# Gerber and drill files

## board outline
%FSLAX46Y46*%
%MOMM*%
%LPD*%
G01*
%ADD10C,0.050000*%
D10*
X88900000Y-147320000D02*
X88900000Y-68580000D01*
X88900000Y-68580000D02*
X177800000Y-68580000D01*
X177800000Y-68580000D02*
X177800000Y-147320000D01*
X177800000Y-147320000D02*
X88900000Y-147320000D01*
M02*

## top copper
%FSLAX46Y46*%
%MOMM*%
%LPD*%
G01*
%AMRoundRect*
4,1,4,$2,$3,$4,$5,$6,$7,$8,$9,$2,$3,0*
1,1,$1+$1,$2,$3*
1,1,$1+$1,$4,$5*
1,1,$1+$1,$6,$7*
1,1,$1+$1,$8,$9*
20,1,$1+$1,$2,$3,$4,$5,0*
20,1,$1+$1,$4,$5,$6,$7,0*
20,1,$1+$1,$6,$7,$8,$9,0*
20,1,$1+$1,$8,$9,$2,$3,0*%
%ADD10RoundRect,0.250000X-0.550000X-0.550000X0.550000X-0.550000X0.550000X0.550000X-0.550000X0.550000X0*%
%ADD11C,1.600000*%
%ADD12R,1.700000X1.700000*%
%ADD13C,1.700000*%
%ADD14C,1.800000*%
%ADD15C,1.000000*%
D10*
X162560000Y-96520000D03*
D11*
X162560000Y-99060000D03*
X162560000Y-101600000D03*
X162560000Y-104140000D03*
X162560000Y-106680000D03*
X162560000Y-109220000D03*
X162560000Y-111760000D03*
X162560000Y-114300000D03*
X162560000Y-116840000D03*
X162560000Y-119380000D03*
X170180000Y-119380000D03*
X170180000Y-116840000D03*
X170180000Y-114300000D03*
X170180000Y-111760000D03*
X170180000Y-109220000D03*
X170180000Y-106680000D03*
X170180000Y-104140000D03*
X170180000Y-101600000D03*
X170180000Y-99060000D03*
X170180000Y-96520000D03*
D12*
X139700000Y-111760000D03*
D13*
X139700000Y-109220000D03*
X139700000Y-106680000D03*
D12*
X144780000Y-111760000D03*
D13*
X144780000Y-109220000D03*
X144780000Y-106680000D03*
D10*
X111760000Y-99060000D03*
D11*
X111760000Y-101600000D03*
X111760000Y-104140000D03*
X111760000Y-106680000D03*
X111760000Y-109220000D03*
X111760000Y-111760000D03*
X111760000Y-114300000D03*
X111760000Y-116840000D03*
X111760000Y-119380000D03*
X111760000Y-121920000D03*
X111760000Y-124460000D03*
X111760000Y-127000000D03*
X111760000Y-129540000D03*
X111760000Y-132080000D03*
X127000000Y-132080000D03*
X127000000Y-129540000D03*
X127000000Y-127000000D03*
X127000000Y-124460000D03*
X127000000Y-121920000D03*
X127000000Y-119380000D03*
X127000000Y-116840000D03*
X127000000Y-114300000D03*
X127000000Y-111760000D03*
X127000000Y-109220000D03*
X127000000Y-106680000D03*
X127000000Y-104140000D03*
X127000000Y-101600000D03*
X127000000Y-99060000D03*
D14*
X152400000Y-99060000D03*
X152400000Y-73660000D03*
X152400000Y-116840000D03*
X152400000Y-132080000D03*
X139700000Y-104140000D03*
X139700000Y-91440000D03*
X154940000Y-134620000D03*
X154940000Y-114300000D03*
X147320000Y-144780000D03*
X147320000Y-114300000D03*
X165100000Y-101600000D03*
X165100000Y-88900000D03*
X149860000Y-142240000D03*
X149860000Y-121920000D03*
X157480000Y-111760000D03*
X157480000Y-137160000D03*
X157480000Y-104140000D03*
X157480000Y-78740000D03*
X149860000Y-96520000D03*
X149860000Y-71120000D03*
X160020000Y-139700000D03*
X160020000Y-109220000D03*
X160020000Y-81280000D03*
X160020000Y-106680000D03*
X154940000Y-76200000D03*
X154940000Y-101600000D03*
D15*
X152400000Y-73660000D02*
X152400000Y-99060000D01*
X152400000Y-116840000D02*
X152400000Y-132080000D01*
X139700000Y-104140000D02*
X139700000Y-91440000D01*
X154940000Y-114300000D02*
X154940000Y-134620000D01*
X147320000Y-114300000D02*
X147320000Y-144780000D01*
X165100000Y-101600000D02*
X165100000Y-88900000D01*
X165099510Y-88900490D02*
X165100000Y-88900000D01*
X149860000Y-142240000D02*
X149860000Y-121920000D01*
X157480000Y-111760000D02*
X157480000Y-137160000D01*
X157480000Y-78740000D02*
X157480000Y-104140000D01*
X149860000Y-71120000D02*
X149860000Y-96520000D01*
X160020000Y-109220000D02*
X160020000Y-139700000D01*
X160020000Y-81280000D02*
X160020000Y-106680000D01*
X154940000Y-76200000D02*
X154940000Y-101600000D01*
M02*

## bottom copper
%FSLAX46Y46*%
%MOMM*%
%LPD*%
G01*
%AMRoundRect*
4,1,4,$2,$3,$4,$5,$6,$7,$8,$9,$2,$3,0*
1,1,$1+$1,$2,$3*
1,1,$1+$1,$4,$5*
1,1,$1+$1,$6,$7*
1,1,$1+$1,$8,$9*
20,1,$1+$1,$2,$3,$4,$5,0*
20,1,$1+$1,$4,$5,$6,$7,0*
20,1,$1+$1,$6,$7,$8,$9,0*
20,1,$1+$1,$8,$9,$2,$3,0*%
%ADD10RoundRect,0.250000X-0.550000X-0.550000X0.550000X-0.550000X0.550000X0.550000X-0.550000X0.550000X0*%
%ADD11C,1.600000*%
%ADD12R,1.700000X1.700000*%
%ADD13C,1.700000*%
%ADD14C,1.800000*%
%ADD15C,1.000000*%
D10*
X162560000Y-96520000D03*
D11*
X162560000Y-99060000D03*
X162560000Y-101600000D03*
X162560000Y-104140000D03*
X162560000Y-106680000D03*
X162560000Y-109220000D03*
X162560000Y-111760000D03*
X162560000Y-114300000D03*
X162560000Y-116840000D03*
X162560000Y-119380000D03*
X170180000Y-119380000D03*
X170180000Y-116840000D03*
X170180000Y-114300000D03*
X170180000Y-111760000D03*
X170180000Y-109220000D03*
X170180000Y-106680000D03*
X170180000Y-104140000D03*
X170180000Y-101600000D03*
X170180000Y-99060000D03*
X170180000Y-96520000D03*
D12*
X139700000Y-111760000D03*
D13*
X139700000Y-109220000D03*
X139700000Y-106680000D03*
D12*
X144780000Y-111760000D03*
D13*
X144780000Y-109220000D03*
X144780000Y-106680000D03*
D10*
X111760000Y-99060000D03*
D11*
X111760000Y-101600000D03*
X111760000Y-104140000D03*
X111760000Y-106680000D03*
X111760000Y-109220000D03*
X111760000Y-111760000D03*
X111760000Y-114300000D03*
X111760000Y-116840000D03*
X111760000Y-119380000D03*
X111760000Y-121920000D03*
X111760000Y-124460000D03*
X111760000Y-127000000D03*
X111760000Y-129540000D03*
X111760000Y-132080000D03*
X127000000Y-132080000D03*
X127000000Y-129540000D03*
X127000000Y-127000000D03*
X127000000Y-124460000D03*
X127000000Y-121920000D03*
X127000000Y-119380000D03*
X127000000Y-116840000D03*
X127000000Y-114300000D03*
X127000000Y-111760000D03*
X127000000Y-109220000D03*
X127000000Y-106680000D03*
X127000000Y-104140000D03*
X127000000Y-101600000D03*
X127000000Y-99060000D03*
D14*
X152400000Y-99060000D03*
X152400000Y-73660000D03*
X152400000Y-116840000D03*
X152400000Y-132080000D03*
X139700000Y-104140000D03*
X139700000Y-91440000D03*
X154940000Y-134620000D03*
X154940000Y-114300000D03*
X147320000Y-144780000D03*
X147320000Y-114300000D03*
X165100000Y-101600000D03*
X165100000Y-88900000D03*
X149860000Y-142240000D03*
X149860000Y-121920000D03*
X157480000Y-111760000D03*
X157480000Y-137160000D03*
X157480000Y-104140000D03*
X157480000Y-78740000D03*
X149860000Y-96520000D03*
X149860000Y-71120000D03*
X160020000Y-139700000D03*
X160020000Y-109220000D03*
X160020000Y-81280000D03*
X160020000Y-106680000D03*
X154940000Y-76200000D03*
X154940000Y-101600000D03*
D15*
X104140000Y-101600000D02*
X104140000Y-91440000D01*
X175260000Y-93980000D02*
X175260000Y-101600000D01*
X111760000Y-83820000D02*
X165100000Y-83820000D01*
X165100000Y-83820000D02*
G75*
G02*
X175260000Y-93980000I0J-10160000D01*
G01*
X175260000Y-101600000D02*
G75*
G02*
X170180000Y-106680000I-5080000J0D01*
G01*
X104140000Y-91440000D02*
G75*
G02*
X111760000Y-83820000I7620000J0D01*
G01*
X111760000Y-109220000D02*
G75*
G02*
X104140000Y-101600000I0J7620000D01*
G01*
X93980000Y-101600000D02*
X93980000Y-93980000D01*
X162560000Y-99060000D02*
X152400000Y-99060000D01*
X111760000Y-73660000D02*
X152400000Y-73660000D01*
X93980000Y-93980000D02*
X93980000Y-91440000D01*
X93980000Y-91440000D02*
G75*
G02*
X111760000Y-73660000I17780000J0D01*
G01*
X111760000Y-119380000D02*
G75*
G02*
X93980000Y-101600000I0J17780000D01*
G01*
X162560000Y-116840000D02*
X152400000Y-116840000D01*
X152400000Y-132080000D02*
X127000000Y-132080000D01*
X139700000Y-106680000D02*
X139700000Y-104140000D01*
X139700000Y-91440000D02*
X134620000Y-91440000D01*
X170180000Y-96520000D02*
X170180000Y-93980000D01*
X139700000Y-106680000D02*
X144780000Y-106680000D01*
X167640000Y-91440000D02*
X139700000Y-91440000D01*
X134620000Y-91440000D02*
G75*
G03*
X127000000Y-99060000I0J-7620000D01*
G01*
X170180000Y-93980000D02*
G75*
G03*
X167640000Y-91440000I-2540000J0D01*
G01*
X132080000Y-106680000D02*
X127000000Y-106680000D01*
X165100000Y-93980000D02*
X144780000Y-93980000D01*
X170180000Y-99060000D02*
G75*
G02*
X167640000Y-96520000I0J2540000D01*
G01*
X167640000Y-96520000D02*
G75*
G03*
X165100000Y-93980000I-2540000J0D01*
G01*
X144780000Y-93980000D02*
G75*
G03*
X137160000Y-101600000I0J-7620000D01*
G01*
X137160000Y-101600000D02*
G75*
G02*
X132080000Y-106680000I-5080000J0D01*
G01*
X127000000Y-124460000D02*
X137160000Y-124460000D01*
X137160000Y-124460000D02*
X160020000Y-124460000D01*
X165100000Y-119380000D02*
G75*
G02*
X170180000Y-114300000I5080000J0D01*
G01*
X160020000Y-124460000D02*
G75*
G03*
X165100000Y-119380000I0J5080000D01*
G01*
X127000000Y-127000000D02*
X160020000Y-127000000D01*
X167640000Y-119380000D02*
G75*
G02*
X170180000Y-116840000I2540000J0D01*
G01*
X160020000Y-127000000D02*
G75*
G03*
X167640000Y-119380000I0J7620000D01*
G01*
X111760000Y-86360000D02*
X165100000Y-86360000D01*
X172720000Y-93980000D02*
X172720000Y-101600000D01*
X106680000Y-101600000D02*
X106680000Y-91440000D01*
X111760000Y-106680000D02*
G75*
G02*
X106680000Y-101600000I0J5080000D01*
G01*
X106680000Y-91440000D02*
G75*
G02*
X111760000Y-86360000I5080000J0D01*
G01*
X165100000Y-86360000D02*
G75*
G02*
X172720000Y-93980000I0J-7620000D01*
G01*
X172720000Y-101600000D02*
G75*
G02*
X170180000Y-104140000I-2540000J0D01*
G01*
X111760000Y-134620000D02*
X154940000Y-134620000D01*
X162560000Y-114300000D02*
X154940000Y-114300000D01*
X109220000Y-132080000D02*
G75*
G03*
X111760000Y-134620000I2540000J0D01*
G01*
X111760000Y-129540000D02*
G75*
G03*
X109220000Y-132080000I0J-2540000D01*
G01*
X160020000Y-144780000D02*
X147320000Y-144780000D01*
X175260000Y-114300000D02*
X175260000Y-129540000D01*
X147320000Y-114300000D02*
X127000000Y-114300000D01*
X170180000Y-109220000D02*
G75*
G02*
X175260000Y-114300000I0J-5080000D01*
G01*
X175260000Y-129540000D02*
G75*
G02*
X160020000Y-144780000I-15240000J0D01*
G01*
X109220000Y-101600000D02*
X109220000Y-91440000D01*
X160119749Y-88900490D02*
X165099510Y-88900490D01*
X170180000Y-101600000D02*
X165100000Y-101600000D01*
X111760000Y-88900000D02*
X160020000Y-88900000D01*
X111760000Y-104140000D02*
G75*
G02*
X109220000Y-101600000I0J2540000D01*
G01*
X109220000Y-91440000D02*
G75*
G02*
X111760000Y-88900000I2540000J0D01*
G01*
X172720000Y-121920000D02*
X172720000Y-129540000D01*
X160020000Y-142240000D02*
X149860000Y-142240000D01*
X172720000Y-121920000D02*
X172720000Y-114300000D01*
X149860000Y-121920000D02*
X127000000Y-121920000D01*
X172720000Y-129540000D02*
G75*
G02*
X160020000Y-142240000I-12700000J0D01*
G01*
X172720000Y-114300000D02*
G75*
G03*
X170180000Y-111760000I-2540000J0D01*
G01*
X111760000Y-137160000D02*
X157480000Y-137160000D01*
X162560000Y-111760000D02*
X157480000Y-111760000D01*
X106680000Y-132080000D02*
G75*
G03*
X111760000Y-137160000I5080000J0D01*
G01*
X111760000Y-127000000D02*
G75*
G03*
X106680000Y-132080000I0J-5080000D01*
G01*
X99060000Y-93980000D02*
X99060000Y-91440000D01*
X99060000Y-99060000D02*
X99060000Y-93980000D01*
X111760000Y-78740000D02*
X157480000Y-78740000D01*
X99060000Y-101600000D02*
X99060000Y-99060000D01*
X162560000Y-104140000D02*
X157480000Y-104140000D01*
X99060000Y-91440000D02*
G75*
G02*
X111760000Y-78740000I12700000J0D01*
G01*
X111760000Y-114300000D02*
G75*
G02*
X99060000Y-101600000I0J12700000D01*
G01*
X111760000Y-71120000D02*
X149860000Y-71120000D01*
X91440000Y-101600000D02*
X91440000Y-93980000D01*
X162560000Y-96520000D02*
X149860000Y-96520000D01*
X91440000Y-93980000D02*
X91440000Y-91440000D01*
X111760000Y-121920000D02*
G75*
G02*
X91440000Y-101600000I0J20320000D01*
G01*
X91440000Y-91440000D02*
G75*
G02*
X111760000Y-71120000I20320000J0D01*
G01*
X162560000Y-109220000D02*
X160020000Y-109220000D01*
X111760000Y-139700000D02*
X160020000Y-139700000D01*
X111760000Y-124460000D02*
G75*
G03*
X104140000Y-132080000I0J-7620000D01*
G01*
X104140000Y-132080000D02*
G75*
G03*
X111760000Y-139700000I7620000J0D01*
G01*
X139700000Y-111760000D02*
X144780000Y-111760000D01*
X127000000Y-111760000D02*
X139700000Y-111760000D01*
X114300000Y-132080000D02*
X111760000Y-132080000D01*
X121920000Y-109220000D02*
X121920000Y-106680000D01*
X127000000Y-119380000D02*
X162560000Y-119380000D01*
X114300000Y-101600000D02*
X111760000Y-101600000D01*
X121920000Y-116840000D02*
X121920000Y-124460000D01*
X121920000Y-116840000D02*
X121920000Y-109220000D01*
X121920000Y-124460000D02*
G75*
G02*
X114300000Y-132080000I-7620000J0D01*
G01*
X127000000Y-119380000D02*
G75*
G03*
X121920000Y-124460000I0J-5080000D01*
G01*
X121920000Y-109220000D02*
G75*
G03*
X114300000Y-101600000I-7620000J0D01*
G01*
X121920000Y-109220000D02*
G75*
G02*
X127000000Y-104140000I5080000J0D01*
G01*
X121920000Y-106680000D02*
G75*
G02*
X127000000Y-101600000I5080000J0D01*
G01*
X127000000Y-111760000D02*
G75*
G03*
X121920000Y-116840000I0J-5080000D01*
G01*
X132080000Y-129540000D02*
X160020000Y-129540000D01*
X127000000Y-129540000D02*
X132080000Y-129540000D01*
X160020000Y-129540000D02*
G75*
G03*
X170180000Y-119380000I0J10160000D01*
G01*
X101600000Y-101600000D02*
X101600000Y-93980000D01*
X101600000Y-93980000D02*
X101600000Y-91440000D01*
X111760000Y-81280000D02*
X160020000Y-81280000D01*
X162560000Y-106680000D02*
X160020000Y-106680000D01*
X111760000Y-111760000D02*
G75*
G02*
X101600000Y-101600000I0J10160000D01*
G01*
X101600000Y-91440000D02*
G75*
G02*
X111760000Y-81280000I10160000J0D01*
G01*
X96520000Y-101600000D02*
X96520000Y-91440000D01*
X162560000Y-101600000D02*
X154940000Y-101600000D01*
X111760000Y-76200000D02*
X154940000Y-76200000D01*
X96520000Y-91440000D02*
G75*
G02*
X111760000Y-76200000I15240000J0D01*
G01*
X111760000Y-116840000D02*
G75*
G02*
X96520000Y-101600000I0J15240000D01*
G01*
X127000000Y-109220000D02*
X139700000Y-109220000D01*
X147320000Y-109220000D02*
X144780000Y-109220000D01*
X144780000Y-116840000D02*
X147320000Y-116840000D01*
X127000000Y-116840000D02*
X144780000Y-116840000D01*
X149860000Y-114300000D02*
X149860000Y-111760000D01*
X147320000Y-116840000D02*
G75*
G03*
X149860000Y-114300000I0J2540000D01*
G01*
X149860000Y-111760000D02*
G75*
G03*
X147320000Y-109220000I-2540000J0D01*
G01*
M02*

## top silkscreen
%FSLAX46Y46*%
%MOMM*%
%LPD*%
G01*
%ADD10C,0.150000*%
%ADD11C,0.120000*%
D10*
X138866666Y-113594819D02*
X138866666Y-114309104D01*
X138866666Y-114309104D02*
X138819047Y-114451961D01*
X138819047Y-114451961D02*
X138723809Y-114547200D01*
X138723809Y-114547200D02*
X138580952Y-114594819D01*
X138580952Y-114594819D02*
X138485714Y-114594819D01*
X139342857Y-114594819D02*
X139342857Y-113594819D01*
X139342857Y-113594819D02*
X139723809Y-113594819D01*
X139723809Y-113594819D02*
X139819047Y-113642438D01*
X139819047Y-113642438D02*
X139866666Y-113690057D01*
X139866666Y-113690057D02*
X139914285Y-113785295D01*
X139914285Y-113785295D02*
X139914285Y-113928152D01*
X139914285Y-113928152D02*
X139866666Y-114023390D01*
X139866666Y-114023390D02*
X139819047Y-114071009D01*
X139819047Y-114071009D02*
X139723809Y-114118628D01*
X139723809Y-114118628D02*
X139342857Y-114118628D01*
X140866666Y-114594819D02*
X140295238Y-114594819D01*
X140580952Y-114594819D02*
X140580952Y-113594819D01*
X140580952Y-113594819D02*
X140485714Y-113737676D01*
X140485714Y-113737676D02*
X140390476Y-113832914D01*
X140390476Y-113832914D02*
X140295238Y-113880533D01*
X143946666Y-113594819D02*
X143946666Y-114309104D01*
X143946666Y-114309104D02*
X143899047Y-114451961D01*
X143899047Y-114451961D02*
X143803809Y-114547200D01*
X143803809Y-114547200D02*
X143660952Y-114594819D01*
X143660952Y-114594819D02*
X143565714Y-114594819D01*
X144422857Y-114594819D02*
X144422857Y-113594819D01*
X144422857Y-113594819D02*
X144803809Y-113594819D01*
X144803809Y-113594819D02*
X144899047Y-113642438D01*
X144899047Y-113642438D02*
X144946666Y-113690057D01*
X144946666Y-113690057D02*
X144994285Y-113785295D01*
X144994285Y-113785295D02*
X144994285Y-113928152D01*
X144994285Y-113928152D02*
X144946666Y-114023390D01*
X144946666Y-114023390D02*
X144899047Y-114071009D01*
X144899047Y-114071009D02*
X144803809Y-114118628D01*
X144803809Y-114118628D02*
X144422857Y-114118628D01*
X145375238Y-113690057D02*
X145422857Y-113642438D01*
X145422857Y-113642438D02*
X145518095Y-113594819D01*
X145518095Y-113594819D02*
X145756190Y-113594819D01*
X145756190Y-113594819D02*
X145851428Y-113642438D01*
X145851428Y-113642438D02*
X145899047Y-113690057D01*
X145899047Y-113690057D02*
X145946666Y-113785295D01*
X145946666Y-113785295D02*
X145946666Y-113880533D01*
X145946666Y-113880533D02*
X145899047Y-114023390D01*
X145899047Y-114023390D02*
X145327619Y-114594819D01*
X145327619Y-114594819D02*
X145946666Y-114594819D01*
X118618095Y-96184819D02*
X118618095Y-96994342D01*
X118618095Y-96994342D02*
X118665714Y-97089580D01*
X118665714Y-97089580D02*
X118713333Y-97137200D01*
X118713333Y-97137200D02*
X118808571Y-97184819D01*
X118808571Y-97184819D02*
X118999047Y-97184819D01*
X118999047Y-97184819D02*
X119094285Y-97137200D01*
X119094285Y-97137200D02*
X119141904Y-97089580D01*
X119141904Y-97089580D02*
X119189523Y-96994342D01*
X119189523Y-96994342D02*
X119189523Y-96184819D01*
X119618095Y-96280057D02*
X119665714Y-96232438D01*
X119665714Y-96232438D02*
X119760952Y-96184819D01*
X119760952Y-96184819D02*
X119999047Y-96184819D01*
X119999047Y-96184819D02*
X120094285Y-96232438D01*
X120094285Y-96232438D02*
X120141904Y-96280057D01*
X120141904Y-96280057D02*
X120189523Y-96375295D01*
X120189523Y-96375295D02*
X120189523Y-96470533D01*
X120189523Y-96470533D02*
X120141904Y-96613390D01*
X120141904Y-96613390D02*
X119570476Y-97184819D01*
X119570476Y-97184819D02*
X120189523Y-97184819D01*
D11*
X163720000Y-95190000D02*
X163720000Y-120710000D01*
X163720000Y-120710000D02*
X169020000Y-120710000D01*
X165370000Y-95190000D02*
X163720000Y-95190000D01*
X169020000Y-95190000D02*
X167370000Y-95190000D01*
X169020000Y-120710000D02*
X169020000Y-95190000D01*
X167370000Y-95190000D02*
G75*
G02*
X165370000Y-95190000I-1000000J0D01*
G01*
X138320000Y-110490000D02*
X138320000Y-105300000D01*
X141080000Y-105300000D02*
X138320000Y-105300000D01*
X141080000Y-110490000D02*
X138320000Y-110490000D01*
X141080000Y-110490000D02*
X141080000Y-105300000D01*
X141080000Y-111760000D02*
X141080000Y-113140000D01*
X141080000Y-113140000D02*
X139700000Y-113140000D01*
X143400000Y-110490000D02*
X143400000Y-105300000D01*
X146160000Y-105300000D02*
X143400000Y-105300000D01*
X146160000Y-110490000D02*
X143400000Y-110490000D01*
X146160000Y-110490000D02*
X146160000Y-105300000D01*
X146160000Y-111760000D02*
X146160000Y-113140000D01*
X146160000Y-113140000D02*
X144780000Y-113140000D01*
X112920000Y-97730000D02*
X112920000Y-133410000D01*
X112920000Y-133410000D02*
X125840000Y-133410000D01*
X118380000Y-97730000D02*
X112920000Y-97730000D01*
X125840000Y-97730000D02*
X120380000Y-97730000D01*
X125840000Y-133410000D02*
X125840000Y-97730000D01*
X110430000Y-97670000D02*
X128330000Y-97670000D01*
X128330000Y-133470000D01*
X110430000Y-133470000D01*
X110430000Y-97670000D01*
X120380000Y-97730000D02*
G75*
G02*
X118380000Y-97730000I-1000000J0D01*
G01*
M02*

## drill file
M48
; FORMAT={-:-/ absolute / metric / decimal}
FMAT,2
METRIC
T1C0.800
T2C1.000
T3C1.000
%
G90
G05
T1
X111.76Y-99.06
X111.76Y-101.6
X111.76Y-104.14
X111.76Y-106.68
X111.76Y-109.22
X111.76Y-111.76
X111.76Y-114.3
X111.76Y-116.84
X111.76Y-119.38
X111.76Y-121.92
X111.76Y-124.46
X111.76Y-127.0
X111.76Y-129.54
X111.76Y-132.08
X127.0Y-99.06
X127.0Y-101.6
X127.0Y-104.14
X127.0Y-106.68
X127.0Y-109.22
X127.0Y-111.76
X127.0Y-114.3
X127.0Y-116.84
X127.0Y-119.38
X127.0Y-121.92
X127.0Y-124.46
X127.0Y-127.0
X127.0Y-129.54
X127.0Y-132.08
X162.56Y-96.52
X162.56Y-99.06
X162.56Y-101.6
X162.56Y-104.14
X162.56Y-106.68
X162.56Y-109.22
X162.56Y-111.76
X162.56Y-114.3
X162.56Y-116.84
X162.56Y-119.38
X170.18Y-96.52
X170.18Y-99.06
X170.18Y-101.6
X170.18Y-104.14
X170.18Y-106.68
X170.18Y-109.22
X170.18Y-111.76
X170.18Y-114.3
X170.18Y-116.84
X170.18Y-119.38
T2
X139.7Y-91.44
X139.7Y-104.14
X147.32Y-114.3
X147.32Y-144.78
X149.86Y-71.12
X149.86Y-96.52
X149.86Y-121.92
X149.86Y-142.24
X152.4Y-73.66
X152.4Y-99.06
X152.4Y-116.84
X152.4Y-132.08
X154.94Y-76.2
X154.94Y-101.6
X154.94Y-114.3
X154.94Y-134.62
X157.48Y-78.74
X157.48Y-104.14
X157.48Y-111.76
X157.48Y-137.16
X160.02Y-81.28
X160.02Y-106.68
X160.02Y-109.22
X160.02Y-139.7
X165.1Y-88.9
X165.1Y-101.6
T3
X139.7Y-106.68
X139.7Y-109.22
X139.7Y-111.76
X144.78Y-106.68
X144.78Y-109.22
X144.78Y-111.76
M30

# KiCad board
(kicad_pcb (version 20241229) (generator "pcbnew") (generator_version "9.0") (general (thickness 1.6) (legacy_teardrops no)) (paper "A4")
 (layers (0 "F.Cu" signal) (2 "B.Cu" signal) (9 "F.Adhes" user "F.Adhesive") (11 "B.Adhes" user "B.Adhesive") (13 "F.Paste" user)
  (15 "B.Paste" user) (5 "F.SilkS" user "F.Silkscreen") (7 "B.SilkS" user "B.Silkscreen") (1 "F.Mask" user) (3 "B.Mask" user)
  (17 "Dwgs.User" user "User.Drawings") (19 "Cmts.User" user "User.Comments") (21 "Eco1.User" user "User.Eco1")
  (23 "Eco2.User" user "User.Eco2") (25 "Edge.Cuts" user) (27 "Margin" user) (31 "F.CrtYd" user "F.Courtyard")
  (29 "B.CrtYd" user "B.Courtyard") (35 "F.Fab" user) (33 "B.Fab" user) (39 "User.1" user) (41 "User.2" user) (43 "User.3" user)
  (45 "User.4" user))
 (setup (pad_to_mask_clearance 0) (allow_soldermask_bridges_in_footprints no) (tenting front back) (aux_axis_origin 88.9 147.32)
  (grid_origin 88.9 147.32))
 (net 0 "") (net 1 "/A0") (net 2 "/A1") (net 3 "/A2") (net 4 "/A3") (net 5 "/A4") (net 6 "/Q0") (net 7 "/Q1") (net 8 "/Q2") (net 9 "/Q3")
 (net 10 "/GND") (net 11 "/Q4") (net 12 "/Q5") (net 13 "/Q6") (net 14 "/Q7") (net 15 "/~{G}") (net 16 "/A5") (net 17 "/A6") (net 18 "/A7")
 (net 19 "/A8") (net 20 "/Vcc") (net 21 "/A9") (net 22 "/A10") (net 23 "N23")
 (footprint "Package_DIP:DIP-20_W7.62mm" (layer "F.Cu") (at 162.56 96.52)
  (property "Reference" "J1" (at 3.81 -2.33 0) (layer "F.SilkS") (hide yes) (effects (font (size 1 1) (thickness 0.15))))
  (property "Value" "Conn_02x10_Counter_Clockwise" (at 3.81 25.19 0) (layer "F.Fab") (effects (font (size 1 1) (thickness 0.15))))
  (fp_line (start 1.16 -1.33) (end 1.16 24.19) (stroke (width 0.12) (type solid)) (layer "F.SilkS"))
  (fp_line (start 1.16 24.19) (end 6.46 24.19) (stroke (width 0.12) (type solid)) (layer "F.SilkS"))
  (fp_line (start 2.81 -1.33) (end 1.16 -1.33) (stroke (width 0.12) (type solid)) (layer "F.SilkS"))
  (fp_line (start 6.46 -1.33) (end 4.81 -1.33) (stroke (width 0.12) (type solid)) (layer "F.SilkS"))
  (fp_line (start 6.46 24.19) (end 6.46 -1.33) (stroke (width 0.12) (type solid)) (layer "F.SilkS"))
  (fp_arc (start 4.81 -1.33) (mid 3.81 -0.33) (end 2.81 -1.33) (stroke (width 0.12) (type solid)) (layer "F.SilkS"))
  (pad "1" thru_hole roundrect (at 0 0) (size 1.6 1.6) (drill 0.8) (layers "*.Cu" "*.Mask") (remove_unused_layers no)
   (roundrect_rratio 0.15625) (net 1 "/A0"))
  (pad "2" thru_hole circle (at 0 2.54) (size 1.6 1.6) (drill 0.8) (layers "*.Cu" "*.Mask") (remove_unused_layers no) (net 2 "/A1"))
  (pad "3" thru_hole circle (at 0 5.08) (size 1.6 1.6) (drill 0.8) (layers "*.Cu" "*.Mask") (remove_unused_layers no) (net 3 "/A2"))
  (pad "4" thru_hole circle (at 0 7.62) (size 1.6 1.6) (drill 0.8) (layers "*.Cu" "*.Mask") (remove_unused_layers no) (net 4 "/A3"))
  (pad "5" thru_hole circle (at 0 10.16) (size 1.6 1.6) (drill 0.8) (layers "*.Cu" "*.Mask") (remove_unused_layers no) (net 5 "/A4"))
  (pad "6" thru_hole circle (at 0 12.7) (size 1.6 1.6) (drill 0.8) (layers "*.Cu" "*.Mask") (remove_unused_layers no) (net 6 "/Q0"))
  (pad "7" thru_hole circle (at 0 15.24) (size 1.6 1.6) (drill 0.8) (layers "*.Cu" "*.Mask") (remove_unused_layers no) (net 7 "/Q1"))
  (pad "8" thru_hole circle (at 0 17.78) (size 1.6 1.6) (drill 0.8) (layers "*.Cu" "*.Mask") (remove_unused_layers no) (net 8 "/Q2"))
  (pad "9" thru_hole circle (at 0 20.32) (size 1.6 1.6) (drill 0.8) (layers "*.Cu" "*.Mask") (remove_unused_layers no) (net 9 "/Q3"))
  (pad "10" thru_hole circle (at 0 22.86) (size 1.6 1.6) (drill 0.8) (layers "*.Cu" "*.Mask") (remove_unused_layers no) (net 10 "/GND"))
  (pad "11" thru_hole circle (at 7.62 22.86) (size 1.6 1.6) (drill 0.8) (layers "*.Cu" "*.Mask") (remove_unused_layers no) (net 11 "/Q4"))
  (pad "12" thru_hole circle (at 7.62 20.32) (size 1.6 1.6) (drill 0.8) (layers "*.Cu" "*.Mask") (remove_unused_layers no) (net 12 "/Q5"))
  (pad "13" thru_hole circle (at 7.62 17.78) (size 1.6 1.6) (drill 0.8) (layers "*.Cu" "*.Mask") (remove_unused_layers no) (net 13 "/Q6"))
  (pad "14" thru_hole circle (at 7.62 15.24) (size 1.6 1.6) (drill 0.8) (layers "*.Cu" "*.Mask") (remove_unused_layers no) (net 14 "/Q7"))
  (pad "15" thru_hole circle (at 7.62 12.7) (size 1.6 1.6) (drill 0.8) (layers "*.Cu" "*.Mask") (remove_unused_layers no) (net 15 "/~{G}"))
  (pad "16" thru_hole circle (at 7.62 10.16) (size 1.6 1.6) (drill 0.8) (layers "*.Cu" "*.Mask") (remove_unused_layers no) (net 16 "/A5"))
  (pad "17" thru_hole circle (at 7.62 7.62) (size 1.6 1.6) (drill 0.8) (layers "*.Cu" "*.Mask") (remove_unused_layers no) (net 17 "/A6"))
  (pad "18" thru_hole circle (at 7.62 5.08) (size 1.6 1.6) (drill 0.8) (layers "*.Cu" "*.Mask") (remove_unused_layers no) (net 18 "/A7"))
  (pad "19" thru_hole circle (at 7.62 2.54) (size 1.6 1.6) (drill 0.8) (layers "*.Cu" "*.Mask") (remove_unused_layers no) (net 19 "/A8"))
  (pad "20" thru_hole circle (at 7.62 0) (size 1.6 1.6) (drill 0.8) (layers "*.Cu" "*.Mask") (remove_unused_layers no) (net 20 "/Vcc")))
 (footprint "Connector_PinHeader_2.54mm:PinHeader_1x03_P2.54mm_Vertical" (layer "F.Cu") (at 139.7 111.76 180)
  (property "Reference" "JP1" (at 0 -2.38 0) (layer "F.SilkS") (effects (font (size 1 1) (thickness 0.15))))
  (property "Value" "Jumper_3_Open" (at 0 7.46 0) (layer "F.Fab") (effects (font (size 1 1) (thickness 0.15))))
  (fp_line (start 1.38 1.27) (end 1.38 6.46) (stroke (width 0.12) (type solid)) (layer "F.SilkS"))
  (fp_line (start -1.38 6.46) (end 1.38 6.46) (stroke (width 0.12) (type solid)) (layer "F.SilkS"))
  (fp_line (start -1.38 1.27) (end 1.38 1.27) (stroke (width 0.12) (type solid)) (layer "F.SilkS"))
  (fp_line (start -1.38 1.27) (end -1.38 6.46) (stroke (width 0.12) (type solid)) (layer "F.SilkS"))
  (fp_line (start -1.38 0) (end -1.38 -1.38) (stroke (width 0.12) (type solid)) (layer "F.SilkS"))
  (fp_line (start -1.38 -1.38) (end 0 -1.38) (stroke (width 0.12) (type solid)) (layer "F.SilkS"))
  (pad "1" thru_hole rect (at 0 0 180) (size 1.7 1.7) (drill 1) (layers "*.Cu" "*.Mask") (remove_unused_layers no) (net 10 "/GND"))
  (pad "2" thru_hole circle (at 0 2.54 180) (size 1.7 1.7) (drill 1) (layers "*.Cu" "*.Mask") (remove_unused_layers no) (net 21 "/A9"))
  (pad "3" thru_hole circle (at 0 5.08 180) (size 1.7 1.7) (drill 1) (layers "*.Cu" "*.Mask") (remove_unused_layers no) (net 20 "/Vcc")))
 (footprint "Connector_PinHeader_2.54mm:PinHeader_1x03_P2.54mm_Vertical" (layer "F.Cu") (at 144.78 111.76 180)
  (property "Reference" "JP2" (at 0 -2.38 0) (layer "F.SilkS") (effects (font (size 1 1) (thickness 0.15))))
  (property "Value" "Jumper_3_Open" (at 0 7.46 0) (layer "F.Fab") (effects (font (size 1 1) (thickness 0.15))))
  (fp_line (start 1.38 1.27) (end 1.38 6.46) (stroke (width 0.12) (type solid)) (layer "F.SilkS"))
  (fp_line (start -1.38 6.46) (end 1.38 6.46) (stroke (width 0.12) (type solid)) (layer "F.SilkS"))
  (fp_line (start -1.38 1.27) (end 1.38 1.27) (stroke (width 0.12) (type solid)) (layer "F.SilkS"))
  (fp_line (start -1.38 1.27) (end -1.38 6.46) (stroke (width 0.12) (type solid)) (layer "F.SilkS"))
  (fp_line (start -1.38 0) (end -1.38 -1.38) (stroke (width 0.12) (type solid)) (layer "F.SilkS"))
  (fp_line (start -1.38 -1.38) (end 0 -1.38) (stroke (width 0.12) (type solid)) (layer "F.SilkS"))
  (pad "1" thru_hole rect (at 0 0 180) (size 1.7 1.7) (drill 1) (layers "*.Cu" "*.Mask") (remove_unused_layers no) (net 10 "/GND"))
  (pad "2" thru_hole circle (at 0 2.54 180) (size 1.7 1.7) (drill 1) (layers "*.Cu" "*.Mask") (remove_unused_layers no) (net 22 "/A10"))
  (pad "3" thru_hole circle (at 0 5.08 180) (size 1.7 1.7) (drill 1) (layers "*.Cu" "*.Mask") (remove_unused_layers no) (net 20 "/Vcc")))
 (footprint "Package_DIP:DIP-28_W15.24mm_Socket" (layer "F.Cu") (at 111.76 99.06)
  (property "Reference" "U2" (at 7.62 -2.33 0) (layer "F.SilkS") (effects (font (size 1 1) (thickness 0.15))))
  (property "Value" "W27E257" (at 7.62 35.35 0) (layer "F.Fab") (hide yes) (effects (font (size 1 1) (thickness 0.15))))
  (fp_line (start 1.16 -1.33) (end 1.16 34.35) (stroke (width 0.12) (type solid)) (layer "F.SilkS"))
  (fp_line (start 1.16 34.35) (end 14.08 34.35) (stroke (width 0.12) (type solid)) (layer "F.SilkS"))
  (fp_line (start 6.62 -1.33) (end 1.16 -1.33) (stroke (width 0.12) (type solid)) (layer "F.SilkS"))
  (fp_line (start 14.08 -1.33) (end 8.62 -1.33) (stroke (width 0.12) (type solid)) (layer "F.SilkS"))
  (fp_line (start 14.08 34.35) (end 14.08 -1.33) (stroke (width 0.12) (type solid)) (layer "F.SilkS"))
  (fp_rect (start -1.33 -1.39) (end 16.57 34.41) (stroke (width 0.12) (type solid)) (fill no) (layer "F.SilkS"))
  (fp_arc (start 8.62 -1.33) (mid 7.62 -0.33) (end 6.62 -1.33) (stroke (width 0.12) (type solid)) (layer "F.SilkS"))
  (pad "1" thru_hole roundrect (at 0 0) (size 1.6 1.6) (drill 0.8) (layers "*.Cu" "*.Mask") (remove_unused_layers no)
   (roundrect_rratio 0.15625) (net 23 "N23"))
  (pad "2" thru_hole circle (at 0 2.54) (size 1.6 1.6) (drill 0.8) (layers "*.Cu" "*.Mask") (remove_unused_layers no) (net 10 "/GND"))
  (pad "3" thru_hole circle (at 0 5.08) (size 1.6 1.6) (drill 0.8) (layers "*.Cu" "*.Mask") (remove_unused_layers no) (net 18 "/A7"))
  (pad "4" thru_hole circle (at 0 7.62) (size 1.6 1.6) (drill 0.8) (layers "*.Cu" "*.Mask") (remove_unused_layers no) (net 17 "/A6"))
  (pad "5" thru_hole circle (at 0 10.16) (size 1.6 1.6) (drill 0.8) (layers "*.Cu" "*.Mask") (remove_unused_layers no) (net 16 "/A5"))
  (pad "6" thru_hole circle (at 0 12.7) (size 1.6 1.6) (drill 0.8) (layers "*.Cu" "*.Mask") (remove_unused_layers no) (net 5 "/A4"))
  (pad "7" thru_hole circle (at 0 15.24) (size 1.6 1.6) (drill 0.8) (layers "*.Cu" "*.Mask") (remove_unused_layers no) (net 4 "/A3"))
  (pad "8" thru_hole circle (at 0 17.78) (size 1.6 1.6) (drill 0.8) (layers "*.Cu" "*.Mask") (remove_unused_layers no) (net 3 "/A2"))
  (pad "9" thru_hole circle (at 0 20.32) (size 1.6 1.6) (drill 0.8) (layers "*.Cu" "*.Mask") (remove_unused_layers no) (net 2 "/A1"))
  (pad "10" thru_hole circle (at 0 22.86) (size 1.6 1.6) (drill 0.8) (layers "*.Cu" "*.Mask") (remove_unused_layers no) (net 1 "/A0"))
  (pad "11" thru_hole circle (at 0 25.4) (size 1.6 1.6) (drill 0.8) (layers "*.Cu" "*.Mask") (remove_unused_layers no) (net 6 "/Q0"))
  (pad "12" thru_hole circle (at 0 27.94) (size 1.6 1.6) (drill 0.8) (layers "*.Cu" "*.Mask") (remove_unused_layers no) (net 7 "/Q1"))
  (pad "13" thru_hole circle (at 0 30.48) (size 1.6 1.6) (drill 0.8) (layers "*.Cu" "*.Mask") (remove_unused_layers no) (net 8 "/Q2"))
  (pad "14" thru_hole circle (at 0 33.02) (size 1.6 1.6) (drill 0.8) (layers "*.Cu" "*.Mask") (remove_unused_layers no) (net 10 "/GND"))
  (pad "15" thru_hole circle (at 15.24 33.02) (size 1.6 1.6) (drill 0.8) (layers "*.Cu" "*.Mask") (remove_unused_layers no) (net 9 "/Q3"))
  (pad "16" thru_hole circle (at 15.24 30.48) (size 1.6 1.6) (drill 0.8) (layers "*.Cu" "*.Mask") (remove_unused_layers no) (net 11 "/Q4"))
  (pad "17" thru_hole circle (at 15.24 27.94) (size 1.6 1.6) (drill 0.8) (layers "*.Cu" "*.Mask") (remove_unused_layers no) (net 12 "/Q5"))
  (pad "18" thru_hole circle (at 15.24 25.4) (size 1.6 1.6) (drill 0.8) (layers "*.Cu" "*.Mask") (remove_unused_layers no) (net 13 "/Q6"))
  (pad "19" thru_hole circle (at 15.24 22.86) (size 1.6 1.6) (drill 0.8) (layers "*.Cu" "*.Mask") (remove_unused_layers no) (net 14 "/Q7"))
  (pad "20" thru_hole circle (at 15.24 20.32) (size 1.6 1.6) (drill 0.8) (layers "*.Cu" "*.Mask") (remove_unused_layers no) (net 10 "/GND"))
  (pad "21" thru_hole circle (at 15.24 17.78) (size 1.6 1.6) (drill 0.8) (layers "*.Cu" "*.Mask") (remove_unused_layers no) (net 22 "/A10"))
  (pad "22" thru_hole circle (at 15.24 15.24) (size 1.6 1.6) (drill 0.8) (layers "*.Cu" "*.Mask") (remove_unused_layers no) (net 15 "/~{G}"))
  (pad "23" thru_hole circle (at 15.24 12.7) (size 1.6 1.6) (drill 0.8) (layers "*.Cu" "*.Mask") (remove_unused_layers no) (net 10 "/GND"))
  (pad "24" thru_hole circle (at 15.24 10.16) (size 1.6 1.6) (drill 0.8) (layers "*.Cu" "*.Mask") (remove_unused_layers no) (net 21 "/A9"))
  (pad "25" thru_hole circle (at 15.24 7.62) (size 1.6 1.6) (drill 0.8) (layers "*.Cu" "*.Mask") (remove_unused_layers no) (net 19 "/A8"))
  (pad "26" thru_hole circle (at 15.24 5.08) (size 1.6 1.6) (drill 0.8) (layers "*.Cu" "*.Mask") (remove_unused_layers no) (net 10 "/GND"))
  (pad "27" thru_hole circle (at 15.24 2.54) (size 1.6 1.6) (drill 0.8) (layers "*.Cu" "*.Mask") (remove_unused_layers no) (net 10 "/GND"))
  (pad "28" thru_hole circle (at 15.24 0) (size 1.6 1.6) (drill 0.8) (layers "*.Cu" "*.Mask") (remove_unused_layers no) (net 20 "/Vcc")))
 (gr_line (start 88.9 147.32) (end 88.9 68.58) (stroke (width 0.05) (type default)) (layer "Edge.Cuts"))
 (gr_line (start 88.9 68.58) (end 177.8 68.58) (stroke (width 0.05) (type default)) (layer "Edge.Cuts"))
 (gr_line (start 177.8 68.58) (end 177.8 147.32) (stroke (width 0.05) (type default)) (layer "Edge.Cuts"))
 (gr_line (start 177.8 147.32) (end 88.9 147.32) (stroke (width 0.05) (type default)) (layer "Edge.Cuts"))
 (segment (start 104.14 101.6) (end 104.14 91.44) (width 1) (layer "B.Cu") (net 16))
 (segment (start 175.26 93.98) (end 175.26 101.6) (width 1) (layer "B.Cu") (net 16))
 (segment (start 111.76 83.82) (end 165.1 83.82) (width 1) (layer "B.Cu") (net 16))
 (arc (start 165.1 83.82) (mid 172.284205 86.795795) (end 175.26 93.98) (width 1) (layer "B.Cu") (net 16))
 (arc (start 175.26 101.6) (mid 173.772102 105.192102) (end 170.18 106.68) (width 1) (layer "B.Cu") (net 16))
 (arc (start 104.14 91.44) (mid 106.371846 86.051846) (end 111.76 83.82) (width 1) (layer "B.Cu") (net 16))
 (arc (start 111.76 109.22) (mid 106.371846 106.988154) (end 104.14 101.6) (width 1) (layer "B.Cu") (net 16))
 (segment (start 152.4 73.66) (end 152.4 99.06) (width 1) (layer "F.Cu") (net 2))
 (via (at 152.4 99.06) (size 1.8) (drill 1) (layers "F.Cu" "B.Cu") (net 2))
 (via (at 152.4 73.66) (size 1.8) (drill 1) (layers "F.Cu" "B.Cu") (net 2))
 (segment (start 93.98 101.6) (end 93.98 93.98) (width 1) (layer "B.Cu") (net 2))
 (segment (start 162.56 99.06) (end 152.4 99.06) (width 1) (layer "B.Cu") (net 2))
 (segment (start 111.76 73.66) (end 152.4 73.66) (width 1) (layer "B.Cu") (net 2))
 (segment (start 93.98 93.98) (end 93.98 91.44) (width 1) (layer "B.Cu") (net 2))
 (arc (start 93.98 91.44) (mid 99.187641 78.867641) (end 111.76 73.66) (width 1) (layer "B.Cu") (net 2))
 (arc (start 111.76 119.38) (mid 99.187641 114.172359) (end 93.98 101.6) (width 1) (layer "B.Cu") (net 2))
 (segment (start 152.4 116.84) (end 152.4 132.08) (width 1) (layer "F.Cu") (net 9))
 (via (at 152.4 116.84) (size 1.8) (drill 1) (layers "F.Cu" "B.Cu") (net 9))
 (via (at 152.4 132.08) (size 1.8) (drill 1) (layers "F.Cu" "B.Cu") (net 9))
 (segment (start 162.56 116.84) (end 152.4 116.84) (width 1) (layer "B.Cu") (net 9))
 (segment (start 152.4 132.08) (end 127 132.08) (width 1) (layer "B.Cu") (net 9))
 (segment (start 139.7 104.14) (end 139.7 91.44) (width 1) (layer "F.Cu") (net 20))
 (via (at 139.7 104.14) (size 1.8) (drill 1) (layers "F.Cu" "B.Cu") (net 20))
 (via (at 139.7 91.44) (size 1.8) (drill 1) (layers "F.Cu" "B.Cu") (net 20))
 (segment (start 139.7 106.68) (end 139.7 104.14) (width 1) (layer "B.Cu") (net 20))
 (segment (start 139.7 91.44) (end 134.62 91.44) (width 1) (layer "B.Cu") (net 20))
 (segment (start 170.18 96.52) (end 170.18 93.98) (width 1) (layer "B.Cu") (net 20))
 (segment (start 139.7 106.68) (end 144.78 106.68) (width 1) (layer "B.Cu") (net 20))
 (segment (start 167.64 91.44) (end 139.7 91.44) (width 1) (layer "B.Cu") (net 20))
 (arc (start 134.62 91.44) (mid 129.231846 93.671846) (end 127 99.06) (width 1) (layer "B.Cu") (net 20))
 (arc (start 170.18 93.98) (mid 169.436051 92.183949) (end 167.64 91.44) (width 1) (layer "B.Cu") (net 20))
 (segment (start 132.08 106.68) (end 127 106.68) (width 1) (layer "B.Cu") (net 19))
 (segment (start 165.1 93.98) (end 144.78 93.98) (width 1) (layer "B.Cu") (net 19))
 (arc (start 170.18 99.06) (mid 168.383949 98.316051) (end 167.64 96.52) (width 1) (layer "B.Cu") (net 19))
 (arc (start 167.64 96.52) (mid 166.896051 94.723949) (end 165.1 93.98) (width 1) (layer "B.Cu") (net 19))
 (arc (start 144.78 93.98) (mid 139.391846 96.211846) (end 137.16 101.6) (width 1) (layer "B.Cu") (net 19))
 (arc (start 137.16 101.6) (mid 135.672102 105.192102) (end 132.08 106.68) (width 1) (layer "B.Cu") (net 19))
 (segment (start 127 124.46) (end 137.16 124.46) (width 1) (layer "B.Cu") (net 13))
 (segment (start 137.16 124.46) (end 160.02 124.46) (width 1) (layer "B.Cu") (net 13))
 (arc (start 165.1 119.38) (mid 166.587898 115.787898) (end 170.18 114.3) (width 1) (layer "B.Cu") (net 13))
 (arc (start 160.02 124.46) (mid 163.612102 122.972102) (end 165.1 119.38) (width 1) (layer "B.Cu") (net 13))
 (segment (start 127 127) (end 160.02 127) (width 1) (layer "B.Cu") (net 12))
 (arc (start 167.64 119.38) (mid 168.383949 117.583949) (end 170.18 116.84) (width 1) (layer "B.Cu") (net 12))
 (arc (start 160.02 127) (mid 165.408154 124.768154) (end 167.64 119.38) (width 1) (layer "B.Cu") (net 12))
 (segment (start 111.76 86.36) (end 165.1 86.36) (width 1) (layer "B.Cu") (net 17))
 (segment (start 172.72 93.98) (end 172.72 101.6) (width 1) (layer "B.Cu") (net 17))
 (segment (start 106.68 101.6) (end 106.68 91.44) (width 1) (layer "B.Cu") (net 17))
 (arc (start 111.76 106.68) (mid 108.167898 105.192102) (end 106.68 101.6) (width 1) (layer "B.Cu") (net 17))
 (arc (start 106.68 91.44) (mid 108.167898 87.847898) (end 111.76 86.36) (width 1) (layer "B.Cu") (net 17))
 (arc (start 165.1 86.36) (mid 170.488154 88.591846) (end 172.72 93.98) (width 1) (layer "B.Cu") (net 17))
 (arc (start 172.72 101.6) (mid 171.976051 103.396051) (end 170.18 104.14) (width 1) (layer "B.Cu") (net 17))
 (segment (start 154.94 114.3) (end 154.94 134.62) (width 1) (layer "F.Cu") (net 8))
 (via (at 154.94 134.62) (size 1.8) (drill 1) (layers "F.Cu" "B.Cu") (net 8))
 (via (at 154.94 114.3) (size 1.8) (drill 1) (layers "F.Cu" "B.Cu") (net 8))
 (segment (start 111.76 134.62) (end 154.94 134.62) (width 1) (layer "B.Cu") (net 8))
 (segment (start 162.56 114.3) (end 154.94 114.3) (width 1) (layer "B.Cu") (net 8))
 (arc (start 109.22 132.08) (mid 109.963949 133.876051) (end 111.76 134.62) (width 1) (layer "B.Cu") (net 8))
 (arc (start 111.76 129.54) (mid 109.963949 130.283949) (end 109.22 132.08) (width 1) (layer "B.Cu") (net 8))
 (segment (start 147.32 114.3) (end 147.32 144.78) (width 1) (layer "F.Cu") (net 15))
 (via (at 147.32 144.78) (size 1.8) (drill 1) (layers "F.Cu" "B.Cu") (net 15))
 (via (at 147.32 114.3) (size 1.8) (drill 1) (layers "F.Cu" "B.Cu") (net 15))
 (segment (start 160.02 144.78) (end 147.32 144.78) (width 1) (layer "B.Cu") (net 15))
 (segment (start 175.26 114.3) (end 175.26 129.54) (width 1) (layer "B.Cu") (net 15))
 (segment (start 147.32 114.3) (end 127 114.3) (width 1) (layer "B.Cu") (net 15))
 (arc (start 170.18 109.22) (mid 173.772102 110.707898) (end 175.26 114.3) (width 1) (layer "B.Cu") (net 15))
 (arc (start 175.26 129.54) (mid 170.796307 140.316307) (end 160.02 144.78) (width 1) (layer "B.Cu") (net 15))
 (segment (start 165.1 101.6) (end 165.1 88.9) (width 1) (layer "F.Cu") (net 18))
 (segment (start 165.09951 88.90049) (end 165.1 88.9) (width 1) (layer "F.Cu") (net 18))
 (via (at 165.1 101.6) (size 1.8) (drill 1) (layers "F.Cu" "B.Cu") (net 18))
 (via (at 165.1 88.9) (size 1.8) (drill 1) (layers "F.Cu" "B.Cu") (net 18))
 (segment (start 109.22 101.6) (end 109.22 91.44) (width 1) (layer "B.Cu") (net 18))
 (segment (start 160.119749 88.90049) (end 165.09951 88.90049) (width 1) (layer "B.Cu") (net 18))
 (segment (start 170.18 101.6) (end 165.1 101.6) (width 1) (layer "B.Cu") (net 18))
 (segment (start 111.76 88.9) (end 160.02 88.9) (width 1) (layer "B.Cu") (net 18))
 (arc (start 111.76 104.14) (mid 109.963949 103.396051) (end 109.22 101.6) (width 1) (layer "B.Cu") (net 18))
 (arc (start 109.22 91.44) (mid 109.963949 89.643949) (end 111.76 88.9) (width 1) (layer "B.Cu") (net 18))
 (segment (start 149.86 142.24) (end 149.86 121.92) (width 1) (layer "F.Cu") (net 14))
 (via (at 149.86 142.24) (size 1.8) (drill 1) (layers "F.Cu" "B.Cu") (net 14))
 (via (at 149.86 121.92) (size 1.8) (drill 1) (layers "F.Cu" "B.Cu") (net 14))
 (segment (start 172.72 121.92) (end 172.72 129.54) (width 1) (layer "B.Cu") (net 14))
 (segment (start 160.02 142.24) (end 149.86 142.24) (width 1) (layer "B.Cu") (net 14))
 (segment (start 172.72 121.92) (end 172.72 114.3) (width 1) (layer "B.Cu") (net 14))
 (segment (start 149.86 121.92) (end 127 121.92) (width 1) (layer "B.Cu") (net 14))
 (arc (start 172.72 129.54) (mid 169.000256 138.520256) (end 160.02 142.24) (width 1) (layer "B.Cu") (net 14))
 (arc (start 172.72 114.3) (mid 171.976051 112.503949) (end 170.18 111.76) (width 1) (layer "B.Cu") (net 14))
 (segment (start 157.48 111.76) (end 157.48 137.16) (width 1) (layer "F.Cu") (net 7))
 (via (at 157.48 111.76) (size 1.8) (drill 1) (layers "F.Cu" "B.Cu") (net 7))
 (via (at 157.48 137.16) (size 1.8) (drill 1) (layers "F.Cu" "B.Cu") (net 7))
 (segment (start 111.76 137.16) (end 157.48 137.16) (width 1) (layer "B.Cu") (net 7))
 (segment (start 162.56 111.76) (end 157.48 111.76) (width 1) (layer "B.Cu") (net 7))
 (arc (start 106.68 132.08) (mid 108.167898 135.672102) (end 111.76 137.16) (width 1) (layer "B.Cu") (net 7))
 (arc (start 111.76 127) (mid 108.167898 128.487898) (end 106.68 132.08) (width 1) (layer "B.Cu") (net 7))
 (segment (start 157.48 78.74) (end 157.48 104.14) (width 1) (layer "F.Cu") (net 4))
 (via (at 157.48 104.14) (size 1.8) (drill 1) (layers "F.Cu" "B.Cu") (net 4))
 (via (at 157.48 78.74) (size 1.8) (drill 1) (layers "F.Cu" "B.Cu") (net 4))
 (segment (start 99.06 93.98) (end 99.06 91.44) (width 1) (layer "B.Cu") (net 4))
 (segment (start 99.06 99.06) (end 99.06 93.98) (width 1) (layer "B.Cu") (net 4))
 (segment (start 111.76 78.74) (end 157.48 78.74) (width 1) (layer "B.Cu") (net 4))
 (segment (start 99.06 101.6) (end 99.06 99.06) (width 1) (layer "B.Cu") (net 4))
 (segment (start 162.56 104.14) (end 157.48 104.14) (width 1) (layer "B.Cu") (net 4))
 (arc (start 99.06 91.44) (mid 102.779744 82.459744) (end 111.76 78.74) (width 1) (layer "B.Cu") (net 4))
 (arc (start 111.76 114.3) (mid 102.779744 110.580256) (end 99.06 101.6) (width 1) (layer "B.Cu") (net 4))
 (segment (start 149.86 71.12) (end 149.86 96.52) (width 1) (layer "F.Cu") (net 1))
 (via (at 149.86 96.52) (size 1.8) (drill 1) (layers "F.Cu" "B.Cu") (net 1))
 (via (at 149.86 71.12) (size 1.8) (drill 1) (layers "F.Cu" "B.Cu") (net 1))
 (segment (start 111.76 71.12) (end 149.86 71.12) (width 1) (layer "B.Cu") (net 1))
 (segment (start 91.44 101.6) (end 91.44 93.98) (width 1) (layer "B.Cu") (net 1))
 (segment (start 162.56 96.52) (end 149.86 96.52) (width 1) (layer "B.Cu") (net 1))
 (segment (start 91.44 93.98) (end 91.44 91.44) (width 1) (layer "B.Cu") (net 1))
 (arc (start 111.76 121.92) (mid 97.39159 115.96841) (end 91.44 101.6) (width 1) (layer "B.Cu") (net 1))
 (arc (start 91.44 91.44) (mid 97.39159 77.07159) (end 111.76 71.12) (width 1) (layer "B.Cu") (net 1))
 (segment (start 160.02 109.22) (end 160.02 139.7) (width 1) (layer "F.Cu") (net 6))
 (via (at 160.02 139.7) (size 1.8) (drill 1) (layers "F.Cu" "B.Cu") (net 6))
 (via (at 160.02 109.22) (size 1.8) (drill 1) (layers "F.Cu" "B.Cu") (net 6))
 (segment (start 162.56 109.22) (end 160.02 109.22) (width 1) (layer "B.Cu") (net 6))
 (segment (start 111.76 139.7) (end 160.02 139.7) (width 1) (layer "B.Cu") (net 6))
 (arc (start 111.76 124.46) (mid 106.371846 126.691846) (end 104.14 132.08) (width 1) (layer "B.Cu") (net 6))
 (arc (start 104.14 132.08) (mid 106.371846 137.468154) (end 111.76 139.7) (width 1) (layer "B.Cu") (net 6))
 (segment (start 139.7 111.76) (end 144.78 111.76) (width 1) (layer "B.Cu") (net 10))
 (segment (start 127 111.76) (end 139.7 111.76) (width 1) (layer "B.Cu") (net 10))
 (segment (start 114.3 132.08) (end 111.76 132.08) (width 1) (layer "B.Cu") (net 10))
 (segment (start 121.92 109.22) (end 121.92 106.68) (width 1) (layer "B.Cu") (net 10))
 (segment (start 127 119.38) (end 162.56 119.38) (width 1) (layer "B.Cu") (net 10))
 (segment (start 114.3 101.6) (end 111.76 101.6) (width 1) (layer "B.Cu") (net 10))
 (segment (start 121.92 116.84) (end 121.92 124.46) (width 1) (layer "B.Cu") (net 10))
 (segment (start 121.92 116.84) (end 121.92 109.22) (width 1) (layer "B.Cu") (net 10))
 (arc (start 121.92 124.46) (mid 119.688154 129.848154) (end 114.3 132.08) (width 1) (layer "B.Cu") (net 10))
 (arc (start 127 119.38) (mid 123.407898 120.867898) (end 121.92 124.46) (width 1) (layer "B.Cu") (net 10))
 (arc (start 121.92 109.22) (mid 119.688154 103.831846) (end 114.3 101.6) (width 1) (layer "B.Cu") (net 10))
 (arc (start 121.92 109.22) (mid 123.407898 105.627898) (end 127 104.14) (width 1) (layer "B.Cu") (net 10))
 (arc (start 121.92 106.68) (mid 123.407898 103.087898) (end 127 101.6) (width 1) (layer "B.Cu") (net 10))
 (arc (start 127 111.76) (mid 123.407898 113.247898) (end 121.92 116.84) (width 1) (layer "B.Cu") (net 10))
 (segment (start 132.08 129.54) (end 160.02 129.54) (width 1) (layer "B.Cu") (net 11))
 (segment (start 127 129.54) (end 132.08 129.54) (width 1) (layer "B.Cu") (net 11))
 (arc (start 160.02 129.54) (mid 167.204205 126.564205) (end 170.18 119.38) (width 1) (layer "B.Cu") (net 11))
 (segment (start 160.02 81.28) (end 160.02 106.68) (width 1) (layer "F.Cu") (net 5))
 (via (at 160.02 81.28) (size 1.8) (drill 1) (layers "F.Cu" "B.Cu") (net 5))
 (via (at 160.02 106.68) (size 1.8) (drill 1) (layers "F.Cu" "B.Cu") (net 5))
 (segment (start 101.6 101.6) (end 101.6 93.98) (width 1) (layer "B.Cu") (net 5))
 (segment (start 101.6 93.98) (end 101.6 91.44) (width 1) (layer "B.Cu") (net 5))
 (segment (start 111.76 81.28) (end 160.02 81.28) (width 1) (layer "B.Cu") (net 5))
 (segment (start 162.56 106.68) (end 160.02 106.68) (width 1) (layer "B.Cu") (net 5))
 (arc (start 111.76 111.76) (mid 104.575795 108.784205) (end 101.6 101.6) (width 1) (layer "B.Cu") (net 5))
 (arc (start 101.6 91.44) (mid 104.575795 84.255795) (end 111.76 81.28) (width 1) (layer "B.Cu") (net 5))
 (segment (start 154.94 76.2) (end 154.94 101.6) (width 1) (layer "F.Cu") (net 3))
 (via (at 154.94 76.2) (size 1.8) (drill 1) (layers "F.Cu" "B.Cu") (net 3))
 (via (at 154.94 101.6) (size 1.8) (drill 1) (layers "F.Cu" "B.Cu") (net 3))
 (segment (start 96.52 101.6) (end 96.52 91.44) (width 1) (layer "B.Cu") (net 3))
 (segment (start 162.56 101.6) (end 154.94 101.6) (width 1) (layer "B.Cu") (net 3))
 (segment (start 111.76 76.2) (end 154.94 76.2) (width 1) (layer "B.Cu") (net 3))
 (arc (start 96.52 91.44) (mid 100.983693 80.663693) (end 111.76 76.2) (width 1) (layer "B.Cu") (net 3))
 (arc (start 111.76 116.84) (mid 100.983693 112.376307) (end 96.52 101.6) (width 1) (layer "B.Cu") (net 3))
 (segment (start 127 109.22) (end 139.7 109.22) (width 1) (layer "B.Cu") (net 21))
 (segment (start 147.32 109.22) (end 144.78 109.22) (width 1) (layer "B.Cu") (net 22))
 (segment (start 144.78 116.84) (end 147.32 116.84) (width 1) (layer "B.Cu") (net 22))
 (segment (start 127 116.84) (end 144.78 116.84) (width 1) (layer "B.Cu") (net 22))
 (segment (start 149.86 114.3) (end 149.86 111.76) (width 1) (layer "B.Cu") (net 22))
 (arc (start 147.32 116.84) (mid 149.116051 116.096051) (end 149.86 114.3) (width 1) (layer "B.Cu") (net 22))
 (arc (start 149.86 111.76) (mid 149.116051 109.963949) (end 147.32 109.22) (width 1) (layer "B.Cu") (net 22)))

